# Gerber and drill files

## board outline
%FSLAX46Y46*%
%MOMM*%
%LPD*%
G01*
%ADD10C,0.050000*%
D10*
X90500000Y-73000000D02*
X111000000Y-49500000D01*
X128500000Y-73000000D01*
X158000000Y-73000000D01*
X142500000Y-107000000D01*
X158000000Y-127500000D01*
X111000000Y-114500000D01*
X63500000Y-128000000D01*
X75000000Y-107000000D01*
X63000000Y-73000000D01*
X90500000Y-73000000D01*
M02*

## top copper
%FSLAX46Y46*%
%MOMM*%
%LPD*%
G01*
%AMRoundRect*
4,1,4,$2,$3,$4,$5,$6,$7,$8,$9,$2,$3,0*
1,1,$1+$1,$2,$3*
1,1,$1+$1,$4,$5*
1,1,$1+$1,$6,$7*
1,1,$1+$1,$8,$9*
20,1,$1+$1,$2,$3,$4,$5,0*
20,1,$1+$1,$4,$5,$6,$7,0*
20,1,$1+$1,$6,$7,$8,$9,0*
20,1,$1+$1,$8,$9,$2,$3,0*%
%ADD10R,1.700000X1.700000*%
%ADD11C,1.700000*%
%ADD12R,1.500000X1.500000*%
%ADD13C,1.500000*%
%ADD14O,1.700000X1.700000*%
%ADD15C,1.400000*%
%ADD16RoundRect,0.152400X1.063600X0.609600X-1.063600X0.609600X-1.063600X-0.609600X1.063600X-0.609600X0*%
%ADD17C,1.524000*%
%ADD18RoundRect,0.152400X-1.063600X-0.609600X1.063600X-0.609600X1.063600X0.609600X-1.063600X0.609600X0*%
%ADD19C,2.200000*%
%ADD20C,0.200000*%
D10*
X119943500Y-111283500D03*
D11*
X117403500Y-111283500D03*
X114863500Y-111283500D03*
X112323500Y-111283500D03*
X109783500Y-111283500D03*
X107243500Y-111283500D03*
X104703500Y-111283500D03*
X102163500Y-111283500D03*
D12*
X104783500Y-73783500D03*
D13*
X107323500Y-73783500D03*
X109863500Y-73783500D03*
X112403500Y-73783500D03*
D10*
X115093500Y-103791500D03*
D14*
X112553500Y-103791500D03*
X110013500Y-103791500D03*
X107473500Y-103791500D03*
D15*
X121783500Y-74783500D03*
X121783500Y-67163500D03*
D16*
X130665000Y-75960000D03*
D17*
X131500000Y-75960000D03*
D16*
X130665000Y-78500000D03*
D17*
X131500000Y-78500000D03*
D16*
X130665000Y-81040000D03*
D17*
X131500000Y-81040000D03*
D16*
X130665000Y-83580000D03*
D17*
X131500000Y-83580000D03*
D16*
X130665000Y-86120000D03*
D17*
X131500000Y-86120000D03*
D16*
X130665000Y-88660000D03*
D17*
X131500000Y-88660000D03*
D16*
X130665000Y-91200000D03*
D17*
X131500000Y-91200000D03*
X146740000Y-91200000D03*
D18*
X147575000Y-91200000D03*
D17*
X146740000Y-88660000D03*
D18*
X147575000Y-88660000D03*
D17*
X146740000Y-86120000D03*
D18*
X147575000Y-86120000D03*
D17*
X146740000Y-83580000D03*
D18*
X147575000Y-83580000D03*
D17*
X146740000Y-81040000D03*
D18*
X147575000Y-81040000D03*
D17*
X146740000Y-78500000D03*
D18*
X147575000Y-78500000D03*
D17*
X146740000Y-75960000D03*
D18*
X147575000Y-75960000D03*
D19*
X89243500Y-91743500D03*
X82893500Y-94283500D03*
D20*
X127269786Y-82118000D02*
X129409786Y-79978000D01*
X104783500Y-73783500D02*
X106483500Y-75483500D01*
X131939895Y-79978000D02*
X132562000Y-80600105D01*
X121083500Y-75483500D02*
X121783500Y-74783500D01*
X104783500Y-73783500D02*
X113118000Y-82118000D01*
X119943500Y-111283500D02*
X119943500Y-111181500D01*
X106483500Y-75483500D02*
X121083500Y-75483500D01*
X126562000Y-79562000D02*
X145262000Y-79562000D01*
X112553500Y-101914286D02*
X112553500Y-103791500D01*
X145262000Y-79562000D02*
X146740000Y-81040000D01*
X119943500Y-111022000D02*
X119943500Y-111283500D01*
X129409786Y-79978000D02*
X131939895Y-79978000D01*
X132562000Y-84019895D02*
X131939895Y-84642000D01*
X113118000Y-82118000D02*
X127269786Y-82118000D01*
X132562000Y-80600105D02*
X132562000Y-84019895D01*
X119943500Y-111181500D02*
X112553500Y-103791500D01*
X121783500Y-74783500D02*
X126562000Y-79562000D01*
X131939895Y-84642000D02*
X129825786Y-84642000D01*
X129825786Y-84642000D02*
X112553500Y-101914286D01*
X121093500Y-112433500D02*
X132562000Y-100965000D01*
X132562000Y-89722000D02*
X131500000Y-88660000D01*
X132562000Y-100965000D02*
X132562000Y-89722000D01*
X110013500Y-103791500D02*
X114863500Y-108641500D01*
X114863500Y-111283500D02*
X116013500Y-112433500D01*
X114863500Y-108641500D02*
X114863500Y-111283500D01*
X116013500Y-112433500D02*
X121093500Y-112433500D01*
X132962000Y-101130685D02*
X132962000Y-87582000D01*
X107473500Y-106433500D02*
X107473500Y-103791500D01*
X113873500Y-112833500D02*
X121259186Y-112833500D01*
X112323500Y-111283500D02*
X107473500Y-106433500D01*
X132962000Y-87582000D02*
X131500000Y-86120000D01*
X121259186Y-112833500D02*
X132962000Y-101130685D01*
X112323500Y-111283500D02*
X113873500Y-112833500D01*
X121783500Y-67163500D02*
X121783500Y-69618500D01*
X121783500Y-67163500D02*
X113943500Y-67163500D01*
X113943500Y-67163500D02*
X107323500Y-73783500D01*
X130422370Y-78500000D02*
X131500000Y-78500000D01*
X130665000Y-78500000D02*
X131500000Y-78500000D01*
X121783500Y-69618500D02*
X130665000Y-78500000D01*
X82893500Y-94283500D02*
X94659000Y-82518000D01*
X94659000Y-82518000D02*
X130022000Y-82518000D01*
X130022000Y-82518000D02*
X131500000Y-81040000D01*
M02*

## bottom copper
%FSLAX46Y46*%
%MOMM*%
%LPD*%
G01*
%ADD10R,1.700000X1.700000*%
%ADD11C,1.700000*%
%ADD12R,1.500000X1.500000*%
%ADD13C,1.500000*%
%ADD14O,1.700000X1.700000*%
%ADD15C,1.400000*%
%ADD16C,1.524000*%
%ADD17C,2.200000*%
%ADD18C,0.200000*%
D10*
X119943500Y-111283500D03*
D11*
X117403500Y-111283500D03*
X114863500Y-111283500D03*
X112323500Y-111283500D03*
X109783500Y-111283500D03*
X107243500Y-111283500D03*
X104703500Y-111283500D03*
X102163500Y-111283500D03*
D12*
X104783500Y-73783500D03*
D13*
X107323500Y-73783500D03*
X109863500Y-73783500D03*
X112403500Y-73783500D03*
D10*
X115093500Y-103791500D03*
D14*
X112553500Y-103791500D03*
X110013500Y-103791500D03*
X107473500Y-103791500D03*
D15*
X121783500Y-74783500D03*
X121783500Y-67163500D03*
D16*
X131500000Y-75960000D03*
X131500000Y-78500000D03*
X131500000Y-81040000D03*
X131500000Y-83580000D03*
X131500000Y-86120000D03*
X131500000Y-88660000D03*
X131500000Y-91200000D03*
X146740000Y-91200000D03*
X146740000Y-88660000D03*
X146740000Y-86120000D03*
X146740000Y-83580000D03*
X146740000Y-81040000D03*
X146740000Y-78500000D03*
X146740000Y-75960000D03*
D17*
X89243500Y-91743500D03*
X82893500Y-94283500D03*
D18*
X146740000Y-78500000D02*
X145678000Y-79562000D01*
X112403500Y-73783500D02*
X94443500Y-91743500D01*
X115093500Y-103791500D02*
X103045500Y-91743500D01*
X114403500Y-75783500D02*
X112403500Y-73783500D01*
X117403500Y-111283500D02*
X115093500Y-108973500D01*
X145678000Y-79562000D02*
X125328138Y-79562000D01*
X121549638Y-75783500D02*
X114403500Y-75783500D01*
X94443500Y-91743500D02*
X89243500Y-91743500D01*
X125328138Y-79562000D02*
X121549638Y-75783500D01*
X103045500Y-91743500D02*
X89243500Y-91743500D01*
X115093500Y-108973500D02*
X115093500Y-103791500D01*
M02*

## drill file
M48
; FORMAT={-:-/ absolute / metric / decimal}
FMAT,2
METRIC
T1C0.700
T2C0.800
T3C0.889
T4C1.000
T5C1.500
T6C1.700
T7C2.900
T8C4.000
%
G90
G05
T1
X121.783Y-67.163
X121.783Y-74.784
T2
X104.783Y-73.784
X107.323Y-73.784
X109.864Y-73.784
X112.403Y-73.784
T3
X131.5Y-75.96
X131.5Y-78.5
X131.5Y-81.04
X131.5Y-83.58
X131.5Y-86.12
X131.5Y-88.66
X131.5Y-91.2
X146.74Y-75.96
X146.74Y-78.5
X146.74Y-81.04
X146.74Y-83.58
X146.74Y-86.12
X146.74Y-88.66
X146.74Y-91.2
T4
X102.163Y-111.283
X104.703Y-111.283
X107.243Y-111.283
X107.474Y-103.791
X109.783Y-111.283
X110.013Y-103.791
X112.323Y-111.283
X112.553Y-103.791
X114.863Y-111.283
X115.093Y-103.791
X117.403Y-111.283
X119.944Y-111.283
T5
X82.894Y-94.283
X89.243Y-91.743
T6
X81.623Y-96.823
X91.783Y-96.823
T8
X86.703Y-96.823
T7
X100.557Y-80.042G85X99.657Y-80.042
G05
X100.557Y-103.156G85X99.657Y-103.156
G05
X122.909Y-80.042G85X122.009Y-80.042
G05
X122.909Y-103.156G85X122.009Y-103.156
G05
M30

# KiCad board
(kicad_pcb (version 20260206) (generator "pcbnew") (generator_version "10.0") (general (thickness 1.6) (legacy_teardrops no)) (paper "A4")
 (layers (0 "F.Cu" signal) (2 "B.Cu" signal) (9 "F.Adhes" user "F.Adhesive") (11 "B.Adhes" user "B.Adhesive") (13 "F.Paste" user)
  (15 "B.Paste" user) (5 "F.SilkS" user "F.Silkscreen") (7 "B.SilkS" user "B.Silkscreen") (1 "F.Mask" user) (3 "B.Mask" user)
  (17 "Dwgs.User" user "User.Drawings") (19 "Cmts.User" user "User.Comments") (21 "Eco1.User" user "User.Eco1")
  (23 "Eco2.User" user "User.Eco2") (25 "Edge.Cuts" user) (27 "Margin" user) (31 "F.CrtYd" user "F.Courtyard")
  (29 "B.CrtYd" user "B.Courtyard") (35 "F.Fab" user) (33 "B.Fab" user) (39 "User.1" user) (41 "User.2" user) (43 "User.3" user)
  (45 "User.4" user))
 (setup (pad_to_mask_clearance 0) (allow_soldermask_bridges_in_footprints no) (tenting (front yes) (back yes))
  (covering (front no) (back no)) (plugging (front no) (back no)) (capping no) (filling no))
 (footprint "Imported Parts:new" (layer "F.Cu") (at 83 82.5)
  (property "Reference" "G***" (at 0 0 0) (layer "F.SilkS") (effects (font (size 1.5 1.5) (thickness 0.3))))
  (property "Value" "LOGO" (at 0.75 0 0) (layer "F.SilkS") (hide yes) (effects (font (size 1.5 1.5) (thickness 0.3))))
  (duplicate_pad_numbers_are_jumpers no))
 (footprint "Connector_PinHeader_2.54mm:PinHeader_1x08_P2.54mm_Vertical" (layer "F.Cu") (at 119.9435 111.2835 -90)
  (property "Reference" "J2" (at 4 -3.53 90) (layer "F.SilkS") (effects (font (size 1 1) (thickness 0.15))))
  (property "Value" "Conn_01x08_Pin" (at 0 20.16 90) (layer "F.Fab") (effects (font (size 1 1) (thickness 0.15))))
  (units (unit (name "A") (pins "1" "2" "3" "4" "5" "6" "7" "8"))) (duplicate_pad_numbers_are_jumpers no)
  (pad "1" thru_hole rect (at 0 0 270) (size 1.7 1.7) (drill 1) (layers "*.Cu" "*.Mask") (remove_unused_layers no) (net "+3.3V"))
  (pad "2" thru_hole circle (at 0 2.54 270) (size 1.7 1.7) (drill 1) (layers "*.Cu" "*.Mask") (remove_unused_layers no) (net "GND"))
  (pad "3" thru_hole circle (at 0 5.08 270) (size 1.7 1.7) (drill 1) (layers "*.Cu" "*.Mask") (remove_unused_layers no) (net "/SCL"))
  (pad "4" thru_hole circle (at 0 7.62 270) (size 1.7 1.7) (drill 1) (layers "*.Cu" "*.Mask") (remove_unused_layers no) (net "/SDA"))
  (pad "5" thru_hole circle (at 0 10.16 270) (size 1.7 1.7) (drill 1) (layers "*.Cu" "*.Mask") (remove_unused_layers no)
   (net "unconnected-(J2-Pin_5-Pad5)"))
  (pad "6" thru_hole circle (at 0 12.7 270) (size 1.7 1.7) (drill 1) (layers "*.Cu" "*.Mask") (remove_unused_layers no)
   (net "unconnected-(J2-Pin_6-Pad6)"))
  (pad "7" thru_hole circle (at 0 15.24 270) (size 1.7 1.7) (drill 1) (layers "*.Cu" "*.Mask") (remove_unused_layers no)
   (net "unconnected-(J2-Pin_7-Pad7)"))
  (pad "8" thru_hole circle (at 0 17.78 270) (size 1.7 1.7) (drill 1) (layers "*.Cu" "*.Mask") (remove_unused_layers no)
   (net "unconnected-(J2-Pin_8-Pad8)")))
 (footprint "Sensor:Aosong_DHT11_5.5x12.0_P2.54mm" (layer "F.Cu") (at 104.7835 73.7835 90)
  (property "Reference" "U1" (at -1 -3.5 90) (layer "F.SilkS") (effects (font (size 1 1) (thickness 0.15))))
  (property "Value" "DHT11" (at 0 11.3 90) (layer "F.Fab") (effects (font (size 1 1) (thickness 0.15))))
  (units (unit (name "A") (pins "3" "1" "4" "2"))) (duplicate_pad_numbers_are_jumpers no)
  (pad "1" thru_hole rect (at 0 0 90) (size 1.5 1.5) (drill 0.8) (layers "*.Cu" "*.Mask") (remove_unused_layers no) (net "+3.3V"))
  (pad "2" thru_hole circle (at 0 2.54 90) (size 1.5 1.5) (drill 0.8) (layers "*.Cu" "*.Mask") (remove_unused_layers no) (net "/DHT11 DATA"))
  (pad "3" thru_hole circle (at 0 5.08 90) (size 1.5 1.5) (drill 0.8) (layers "*.Cu" "*.Mask") (remove_unused_layers no)
   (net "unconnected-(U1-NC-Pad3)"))
  (pad "4" thru_hole circle (at 0 7.62 90) (size 1.5 1.5) (drill 0.8) (layers "*.Cu" "*.Mask") (remove_unused_layers no) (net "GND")))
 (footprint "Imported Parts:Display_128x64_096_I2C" (layer "F.Cu") (at 111.2835 103.7915 180)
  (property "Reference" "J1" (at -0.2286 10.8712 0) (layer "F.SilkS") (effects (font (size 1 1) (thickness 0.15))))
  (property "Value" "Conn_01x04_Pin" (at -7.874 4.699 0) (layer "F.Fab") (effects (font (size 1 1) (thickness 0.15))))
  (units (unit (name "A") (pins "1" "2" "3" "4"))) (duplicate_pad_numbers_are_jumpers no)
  (pad "" np_thru_hole oval (at -11.176 0.635 180) (size 3.8 2.9) (drill oval 3.8 2.9) (layers "*.Cu" "*.Mask"))
  (pad "" np_thru_hole oval (at -11.176 23.749 180) (size 3.8 2.9) (drill oval 3.8 2.9) (layers "*.Cu" "*.Mask"))
  (pad "" np_thru_hole oval (at 11.176 0.635 180) (size 3.8 2.9) (drill oval 3.8 2.9) (layers "*.Cu" "*.Mask"))
  (pad "" np_thru_hole oval (at 11.176 23.749 180) (size 3.8 2.9) (drill oval 3.8 2.9) (layers "*.Cu" "*.Mask"))
  (pad "1" thru_hole rect (at -3.81 0 270) (size 1.7 1.7) (drill 1) (layers "*.Cu" "*.Mask") (remove_unused_layers no) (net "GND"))
  (pad "2" thru_hole oval (at -1.27 0 270) (size 1.7 1.7) (drill 1) (layers "*.Cu" "*.Mask") (remove_unused_layers no) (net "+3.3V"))
  (pad "3" thru_hole oval (at 1.27 0 270) (size 1.7 1.7) (drill 1) (layers "*.Cu" "*.Mask") (remove_unused_layers no) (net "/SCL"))
  (pad "4" thru_hole oval (at 3.81 0 270) (size 1.7 1.7) (drill 1) (layers "*.Cu" "*.Mask") (remove_unused_layers no) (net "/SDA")))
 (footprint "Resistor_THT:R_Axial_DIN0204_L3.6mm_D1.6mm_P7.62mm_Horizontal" (layer "F.Cu") (at 121.7835 74.7835 90)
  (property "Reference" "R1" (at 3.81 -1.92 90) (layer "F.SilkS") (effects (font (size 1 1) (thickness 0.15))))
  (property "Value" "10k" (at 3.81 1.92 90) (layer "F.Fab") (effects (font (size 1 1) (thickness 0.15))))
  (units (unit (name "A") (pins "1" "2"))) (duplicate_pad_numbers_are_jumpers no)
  (pad "1" thru_hole circle (at 0 0 90) (size 1.4 1.4) (drill 0.7) (layers "*.Cu" "*.Mask") (remove_unused_layers no) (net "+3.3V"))
  (pad "2" thru_hole circle (at 7.62 0 90) (size 1.4 1.4) (drill 0.7) (layers "*.Cu" "*.Mask") (remove_unused_layers no) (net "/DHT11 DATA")))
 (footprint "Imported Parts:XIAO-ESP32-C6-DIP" (layer "F.Cu") (at 139.12 83.58 90)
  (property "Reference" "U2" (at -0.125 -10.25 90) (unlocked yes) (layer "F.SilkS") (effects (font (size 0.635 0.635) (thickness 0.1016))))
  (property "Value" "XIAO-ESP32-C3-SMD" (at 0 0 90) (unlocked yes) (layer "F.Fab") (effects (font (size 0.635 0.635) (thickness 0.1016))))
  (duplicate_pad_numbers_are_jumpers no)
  (pad "1" smd roundrect (at 7.62 -8.455 180) (size 2.432 1.524) (layers "F.Cu" "F.Mask") (roundrect_rratio 0.1)
   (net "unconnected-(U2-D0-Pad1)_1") (thermal_bridge_angle 45))
  (pad "1" thru_hole circle (at 7.62 -7.62 180) (size 1.524 1.524) (drill 0.889) (layers "*.Cu" "*.Mask") (remove_unused_layers no)
   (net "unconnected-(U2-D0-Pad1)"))
  (pad "2" smd roundrect (at 5.08 -8.455 180) (size 2.432 1.524) (layers "F.Cu" "F.Mask") (roundrect_rratio 0.1) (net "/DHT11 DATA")
   (thermal_bridge_angle 45))
  (pad "2" thru_hole circle (at 5.08 -7.62 180) (size 1.524 1.524) (drill 0.889) (layers "*.Cu" "*.Mask") (remove_unused_layers no)
   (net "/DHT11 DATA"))
  (pad "3" smd roundrect (at 2.54 -8.455 180) (size 2.432 1.524) (layers "F.Cu" "F.Mask") (roundrect_rratio 0.1) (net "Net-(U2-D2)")
   (thermal_bridge_angle 45))
  (pad "3" thru_hole circle (at 2.54 -7.62 180) (size 1.524 1.524) (drill 0.889) (layers "*.Cu" "*.Mask") (remove_unused_layers no)
   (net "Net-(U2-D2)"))
  (pad "4" smd roundrect (at 0 -8.455 180) (size 2.432 1.524) (layers "F.Cu" "F.Mask") (roundrect_rratio 0.1)
   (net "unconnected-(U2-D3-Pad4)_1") (thermal_bridge_angle 45))
  (pad "4" thru_hole circle (at 0 -7.62 180) (size 1.524 1.524) (drill 0.889) (layers "*.Cu" "*.Mask") (remove_unused_layers no)
   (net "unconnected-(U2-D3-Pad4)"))
  (pad "5" smd roundrect (at -2.54 -8.455 180) (size 2.432 1.524) (layers "F.Cu" "F.Mask") (roundrect_rratio 0.1) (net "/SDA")
   (thermal_bridge_angle 45))
  (pad "5" thru_hole circle (at -2.54 -7.62 180) (size 1.524 1.524) (drill 0.889) (layers "*.Cu" "*.Mask") (remove_unused_layers no)
   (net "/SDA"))
  (pad "6" smd roundrect (at -5.08 -8.455 180) (size 2.432 1.524) (layers "F.Cu" "F.Mask") (roundrect_rratio 0.1) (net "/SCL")
   (thermal_bridge_angle 45))
  (pad "6" thru_hole circle (at -5.08 -7.62 180) (size 1.524 1.524) (drill 0.889) (layers "*.Cu" "*.Mask") (remove_unused_layers no)
   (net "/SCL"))
  (pad "7" smd roundrect (at -7.62 -8.455 180) (size 2.432 1.524) (layers "F.Cu" "F.Mask") (roundrect_rratio 0.1)
   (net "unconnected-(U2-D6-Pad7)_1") (thermal_bridge_angle 45))
  (pad "7" thru_hole circle (at -7.62 -7.62 180) (size 1.524 1.524) (drill 0.889) (layers "*.Cu" "*.Mask") (remove_unused_layers no)
   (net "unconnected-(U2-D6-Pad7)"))
  (pad "8" thru_hole circle (at -7.62 7.62) (size 1.524 1.524) (drill 0.889) (layers "*.Cu" "*.Mask") (remove_unused_layers no)
   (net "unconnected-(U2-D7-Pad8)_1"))
  (pad "8" smd roundrect (at -7.62 8.455) (size 2.432 1.524) (layers "F.Cu" "F.Mask") (roundrect_rratio 0.1)
   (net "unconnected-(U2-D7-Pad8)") (thermal_bridge_angle 45))
  (pad "9" thru_hole circle (at -5.08 7.62) (size 1.524 1.524) (drill 0.889) (layers "*.Cu" "*.Mask") (remove_unused_layers no)
   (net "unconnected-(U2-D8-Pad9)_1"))
  (pad "9" smd roundrect (at -5.08 8.455) (size 2.432 1.524) (layers "F.Cu" "F.Mask") (roundrect_rratio 0.1)
   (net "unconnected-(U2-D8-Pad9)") (thermal_bridge_angle 45))
  (pad "10" thru_hole circle (at -2.54 7.62) (size 1.524 1.524) (drill 0.889) (layers "*.Cu" "*.Mask") (remove_unused_layers no)
   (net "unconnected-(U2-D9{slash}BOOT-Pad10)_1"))
  (pad "10" smd roundrect (at -2.54 8.455) (size 2.432 1.524) (layers "F.Cu" "F.Mask") (roundrect_rratio 0.1)
   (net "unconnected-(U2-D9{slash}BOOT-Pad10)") (thermal_bridge_angle 45))
  (pad "11" thru_hole circle (at 0 7.62) (size 1.524 1.524) (drill 0.889) (layers "*.Cu" "*.Mask") (remove_unused_layers no)
   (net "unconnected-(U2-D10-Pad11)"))
  (pad "11" smd roundrect (at 0 8.455) (size 2.432 1.524) (layers "F.Cu" "F.Mask") (roundrect_rratio 0.1)
   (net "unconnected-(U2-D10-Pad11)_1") (thermal_bridge_angle 45))
  (pad "12" thru_hole circle (at 2.54 7.62) (size 1.524 1.524) (drill 0.889) (layers "*.Cu" "*.Mask") (remove_unused_layers no)
   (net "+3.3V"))
  (pad "12" smd roundrect (at 2.54 8.455) (size 2.432 1.524) (layers "F.Cu" "F.Mask") (roundrect_rratio 0.1) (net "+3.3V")
   (thermal_bridge_angle 45))
  (pad "13" thru_hole circle (at 5.08 7.62) (size 1.524 1.524) (drill 0.889) (layers "*.Cu" "*.Mask") (remove_unused_layers no) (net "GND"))
  (pad "13" smd roundrect (at 5.08 8.455) (size 2.432 1.524) (layers "F.Cu" "F.Mask") (roundrect_rratio 0.1) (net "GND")
   (thermal_bridge_angle 45))
  (pad "14" thru_hole circle (at 7.62 7.62) (size 1.524 1.524) (drill 0.889) (layers "*.Cu" "*.Mask") (remove_unused_layers no) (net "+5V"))
  (pad "14" smd roundrect (at 7.62 8.455) (size 2.432 1.524) (layers "F.Cu" "F.Mask") (roundrect_rratio 0.1) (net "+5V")
   (thermal_bridge_angle 45)))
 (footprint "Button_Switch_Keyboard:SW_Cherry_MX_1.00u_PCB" (layer "F.Cu") (at 89.2435 91.7435)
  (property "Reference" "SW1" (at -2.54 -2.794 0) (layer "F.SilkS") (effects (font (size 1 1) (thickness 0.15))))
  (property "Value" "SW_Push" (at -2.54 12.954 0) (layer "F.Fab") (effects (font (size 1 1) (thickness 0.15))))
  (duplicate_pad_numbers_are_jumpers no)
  (pad "" np_thru_hole circle (at -7.62 5.08) (size 1.7 1.7) (drill 1.7) (layers "*.Cu" "*.Mask"))
  (pad "" np_thru_hole circle (at -2.54 5.08) (size 4 4) (drill 4) (layers "*.Cu" "*.Mask"))
  (pad "" np_thru_hole circle (at 2.54 5.08) (size 1.7 1.7) (drill 1.7) (layers "*.Cu" "*.Mask"))
  (pad "1" thru_hole circle (at 0 0) (size 2.2 2.2) (drill 1.5) (layers "*.Cu" "*.Mask") (remove_unused_layers no) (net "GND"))
  (pad "2" thru_hole circle (at -6.35 2.54) (size 2.2 2.2) (drill 1.5) (layers "*.Cu" "*.Mask") (remove_unused_layers no)
   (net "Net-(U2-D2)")))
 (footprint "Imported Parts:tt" (layer "F.Cu") (at 112 62.5)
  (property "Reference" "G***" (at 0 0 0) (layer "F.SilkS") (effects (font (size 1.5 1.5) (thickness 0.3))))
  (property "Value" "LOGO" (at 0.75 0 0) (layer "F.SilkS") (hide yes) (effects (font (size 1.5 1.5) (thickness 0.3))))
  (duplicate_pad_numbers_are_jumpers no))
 (gr_poly
  (pts (xy 90.5 73) (xy 111 49.5) (xy 128.5 73) (xy 158 73) (xy 142.5 107) (xy 158 127.5) (xy 111 114.5) (xy 63.5 128) (xy 75 107)
   (xy 63 73))
  (stroke (width 0.05) (type solid)) (fill no) (layer "Edge.Cuts"))
 (segment (start 127.269786 82.118) (end 129.409786 79.978) (width 0.2) (layer "F.Cu") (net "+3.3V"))
 (segment (start 104.7835 73.7835) (end 106.4835 75.4835) (width 0.2) (layer "F.Cu") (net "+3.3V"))
 (segment (start 131.939895 79.978) (end 132.562 80.600105) (width 0.2) (layer "F.Cu") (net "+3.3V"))
 (segment (start 121.0835 75.4835) (end 121.7835 74.7835) (width 0.2) (layer "F.Cu") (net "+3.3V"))
 (segment (start 104.7835 73.7835) (end 113.118 82.118) (width 0.2) (layer "F.Cu") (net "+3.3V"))
 (segment (start 119.9435 111.2835) (end 119.9435 111.1815) (width 0.2) (layer "F.Cu") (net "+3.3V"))
 (segment (start 106.4835 75.4835) (end 121.0835 75.4835) (width 0.2) (layer "F.Cu") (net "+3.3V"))
 (segment (start 126.562 79.562) (end 145.262 79.562) (width 0.2) (layer "F.Cu") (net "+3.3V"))
 (segment (start 112.5535 101.914286) (end 112.5535 103.7915) (width 0.2) (layer "F.Cu") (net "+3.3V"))
 (segment (start 145.262 79.562) (end 146.74 81.04) (width 0.2) (layer "F.Cu") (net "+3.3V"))
 (segment (start 119.9435 111.022) (end 119.9435 111.2835) (width 0.2) (layer "F.Cu") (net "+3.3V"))
 (segment (start 129.409786 79.978) (end 131.939895 79.978) (width 0.2) (layer "F.Cu") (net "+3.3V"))
 (segment (start 132.562 84.019895) (end 131.939895 84.642) (width 0.2) (layer "F.Cu") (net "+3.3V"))
 (segment (start 113.118 82.118) (end 127.269786 82.118) (width 0.2) (layer "F.Cu") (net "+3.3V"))
 (segment (start 132.562 80.600105) (end 132.562 84.019895) (width 0.2) (layer "F.Cu") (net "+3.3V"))
 (segment (start 119.9435 111.1815) (end 112.5535 103.7915) (width 0.2) (layer "F.Cu") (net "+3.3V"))
 (segment (start 121.7835 74.7835) (end 126.562 79.562) (width 0.2) (layer "F.Cu") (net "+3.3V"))
 (segment (start 131.939895 84.642) (end 129.825786 84.642) (width 0.2) (layer "F.Cu") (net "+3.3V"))
 (segment (start 129.825786 84.642) (end 112.5535 101.914286) (width 0.2) (layer "F.Cu") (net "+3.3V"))
 (segment (start 146.74 78.5) (end 145.678 79.562) (width 0.2) (layer "B.Cu") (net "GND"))
 (segment (start 112.4035 73.7835) (end 94.4435 91.7435) (width 0.2) (layer "B.Cu") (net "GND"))
 (segment (start 115.0935 103.7915) (end 103.0455 91.7435) (width 0.2) (layer "B.Cu") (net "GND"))
 (segment (start 114.4035 75.7835) (end 112.4035 73.7835) (width 0.2) (layer "B.Cu") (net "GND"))
 (segment (start 117.4035 111.2835) (end 115.0935 108.9735) (width 0.2) (layer "B.Cu") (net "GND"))
 (segment (start 145.678 79.562) (end 125.328138 79.562) (width 0.2) (layer "B.Cu") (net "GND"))
 (segment (start 121.549638 75.7835) (end 114.4035 75.7835) (width 0.2) (layer "B.Cu") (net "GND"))
 (segment (start 94.4435 91.7435) (end 89.2435 91.7435) (width 0.2) (layer "B.Cu") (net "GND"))
 (segment (start 125.328138 79.562) (end 121.549638 75.7835) (width 0.2) (layer "B.Cu") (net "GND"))
 (segment (start 103.0455 91.7435) (end 89.2435 91.7435) (width 0.2) (layer "B.Cu") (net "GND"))
 (segment (start 115.0935 108.9735) (end 115.0935 103.7915) (width 0.2) (layer "B.Cu") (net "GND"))
 (segment (start 121.0935 112.4335) (end 132.562 100.965) (width 0.2) (layer "F.Cu") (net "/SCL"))
 (segment (start 132.562 89.722) (end 131.5 88.66) (width 0.2) (layer "F.Cu") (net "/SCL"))
 (segment (start 132.562 100.965) (end 132.562 89.722) (width 0.2) (layer "F.Cu") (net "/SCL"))
 (segment (start 110.0135 103.7915) (end 114.8635 108.6415) (width 0.2) (layer "F.Cu") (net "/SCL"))
 (segment (start 114.8635 111.2835) (end 116.0135 112.4335) (width 0.2) (layer "F.Cu") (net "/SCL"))
 (segment (start 114.8635 108.6415) (end 114.8635 111.2835) (width 0.2) (layer "F.Cu") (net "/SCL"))
 (segment (start 116.0135 112.4335) (end 121.0935 112.4335) (width 0.2) (layer "F.Cu") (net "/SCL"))
 (segment (start 132.962 101.130685) (end 132.962 87.582) (width 0.2) (layer "F.Cu") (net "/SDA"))
 (segment (start 107.4735 106.4335) (end 107.4735 103.7915) (width 0.2) (layer "F.Cu") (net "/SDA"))
 (segment (start 113.8735 112.8335) (end 121.259186 112.8335) (width 0.2) (layer "F.Cu") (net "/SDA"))
 (segment (start 112.3235 111.2835) (end 107.4735 106.4335) (width 0.2) (layer "F.Cu") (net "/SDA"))
 (segment (start 132.962 87.582) (end 131.5 86.12) (width 0.2) (layer "F.Cu") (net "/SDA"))
 (segment (start 121.259186 112.8335) (end 132.962 101.130685) (width 0.2) (layer "F.Cu") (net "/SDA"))
 (segment (start 112.3235 111.2835) (end 113.8735 112.8335) (width 0.2) (layer "F.Cu") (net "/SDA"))
 (segment (start 121.7835 67.1635) (end 121.7835 69.6185) (width 0.2) (layer "F.Cu") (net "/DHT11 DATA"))
 (segment (start 121.7835 67.1635) (end 113.9435 67.1635) (width 0.2) (layer "F.Cu") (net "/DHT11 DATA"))
 (segment (start 113.9435 67.1635) (end 107.3235 73.7835) (width 0.2) (layer "F.Cu") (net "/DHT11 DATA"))
 (segment (start 130.42237 78.5) (end 131.5 78.5) (width 0.2) (layer "F.Cu") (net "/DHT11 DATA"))
 (segment (start 130.665 78.5) (end 131.5 78.5) (width 0.2) (layer "F.Cu") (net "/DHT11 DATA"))
 (segment (start 121.7835 69.6185) (end 130.665 78.5) (width 0.2) (layer "F.Cu") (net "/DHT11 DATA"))
 (segment (start 82.8935 94.2835) (end 94.659 82.518) (width 0.2) (layer "F.Cu") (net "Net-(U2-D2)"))
 (segment (start 94.659 82.518) (end 130.022 82.518) (width 0.2) (layer "F.Cu") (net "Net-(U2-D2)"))
 (segment (start 130.022 82.518) (end 131.5 81.04) (width 0.2) (layer "F.Cu") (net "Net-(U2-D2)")))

